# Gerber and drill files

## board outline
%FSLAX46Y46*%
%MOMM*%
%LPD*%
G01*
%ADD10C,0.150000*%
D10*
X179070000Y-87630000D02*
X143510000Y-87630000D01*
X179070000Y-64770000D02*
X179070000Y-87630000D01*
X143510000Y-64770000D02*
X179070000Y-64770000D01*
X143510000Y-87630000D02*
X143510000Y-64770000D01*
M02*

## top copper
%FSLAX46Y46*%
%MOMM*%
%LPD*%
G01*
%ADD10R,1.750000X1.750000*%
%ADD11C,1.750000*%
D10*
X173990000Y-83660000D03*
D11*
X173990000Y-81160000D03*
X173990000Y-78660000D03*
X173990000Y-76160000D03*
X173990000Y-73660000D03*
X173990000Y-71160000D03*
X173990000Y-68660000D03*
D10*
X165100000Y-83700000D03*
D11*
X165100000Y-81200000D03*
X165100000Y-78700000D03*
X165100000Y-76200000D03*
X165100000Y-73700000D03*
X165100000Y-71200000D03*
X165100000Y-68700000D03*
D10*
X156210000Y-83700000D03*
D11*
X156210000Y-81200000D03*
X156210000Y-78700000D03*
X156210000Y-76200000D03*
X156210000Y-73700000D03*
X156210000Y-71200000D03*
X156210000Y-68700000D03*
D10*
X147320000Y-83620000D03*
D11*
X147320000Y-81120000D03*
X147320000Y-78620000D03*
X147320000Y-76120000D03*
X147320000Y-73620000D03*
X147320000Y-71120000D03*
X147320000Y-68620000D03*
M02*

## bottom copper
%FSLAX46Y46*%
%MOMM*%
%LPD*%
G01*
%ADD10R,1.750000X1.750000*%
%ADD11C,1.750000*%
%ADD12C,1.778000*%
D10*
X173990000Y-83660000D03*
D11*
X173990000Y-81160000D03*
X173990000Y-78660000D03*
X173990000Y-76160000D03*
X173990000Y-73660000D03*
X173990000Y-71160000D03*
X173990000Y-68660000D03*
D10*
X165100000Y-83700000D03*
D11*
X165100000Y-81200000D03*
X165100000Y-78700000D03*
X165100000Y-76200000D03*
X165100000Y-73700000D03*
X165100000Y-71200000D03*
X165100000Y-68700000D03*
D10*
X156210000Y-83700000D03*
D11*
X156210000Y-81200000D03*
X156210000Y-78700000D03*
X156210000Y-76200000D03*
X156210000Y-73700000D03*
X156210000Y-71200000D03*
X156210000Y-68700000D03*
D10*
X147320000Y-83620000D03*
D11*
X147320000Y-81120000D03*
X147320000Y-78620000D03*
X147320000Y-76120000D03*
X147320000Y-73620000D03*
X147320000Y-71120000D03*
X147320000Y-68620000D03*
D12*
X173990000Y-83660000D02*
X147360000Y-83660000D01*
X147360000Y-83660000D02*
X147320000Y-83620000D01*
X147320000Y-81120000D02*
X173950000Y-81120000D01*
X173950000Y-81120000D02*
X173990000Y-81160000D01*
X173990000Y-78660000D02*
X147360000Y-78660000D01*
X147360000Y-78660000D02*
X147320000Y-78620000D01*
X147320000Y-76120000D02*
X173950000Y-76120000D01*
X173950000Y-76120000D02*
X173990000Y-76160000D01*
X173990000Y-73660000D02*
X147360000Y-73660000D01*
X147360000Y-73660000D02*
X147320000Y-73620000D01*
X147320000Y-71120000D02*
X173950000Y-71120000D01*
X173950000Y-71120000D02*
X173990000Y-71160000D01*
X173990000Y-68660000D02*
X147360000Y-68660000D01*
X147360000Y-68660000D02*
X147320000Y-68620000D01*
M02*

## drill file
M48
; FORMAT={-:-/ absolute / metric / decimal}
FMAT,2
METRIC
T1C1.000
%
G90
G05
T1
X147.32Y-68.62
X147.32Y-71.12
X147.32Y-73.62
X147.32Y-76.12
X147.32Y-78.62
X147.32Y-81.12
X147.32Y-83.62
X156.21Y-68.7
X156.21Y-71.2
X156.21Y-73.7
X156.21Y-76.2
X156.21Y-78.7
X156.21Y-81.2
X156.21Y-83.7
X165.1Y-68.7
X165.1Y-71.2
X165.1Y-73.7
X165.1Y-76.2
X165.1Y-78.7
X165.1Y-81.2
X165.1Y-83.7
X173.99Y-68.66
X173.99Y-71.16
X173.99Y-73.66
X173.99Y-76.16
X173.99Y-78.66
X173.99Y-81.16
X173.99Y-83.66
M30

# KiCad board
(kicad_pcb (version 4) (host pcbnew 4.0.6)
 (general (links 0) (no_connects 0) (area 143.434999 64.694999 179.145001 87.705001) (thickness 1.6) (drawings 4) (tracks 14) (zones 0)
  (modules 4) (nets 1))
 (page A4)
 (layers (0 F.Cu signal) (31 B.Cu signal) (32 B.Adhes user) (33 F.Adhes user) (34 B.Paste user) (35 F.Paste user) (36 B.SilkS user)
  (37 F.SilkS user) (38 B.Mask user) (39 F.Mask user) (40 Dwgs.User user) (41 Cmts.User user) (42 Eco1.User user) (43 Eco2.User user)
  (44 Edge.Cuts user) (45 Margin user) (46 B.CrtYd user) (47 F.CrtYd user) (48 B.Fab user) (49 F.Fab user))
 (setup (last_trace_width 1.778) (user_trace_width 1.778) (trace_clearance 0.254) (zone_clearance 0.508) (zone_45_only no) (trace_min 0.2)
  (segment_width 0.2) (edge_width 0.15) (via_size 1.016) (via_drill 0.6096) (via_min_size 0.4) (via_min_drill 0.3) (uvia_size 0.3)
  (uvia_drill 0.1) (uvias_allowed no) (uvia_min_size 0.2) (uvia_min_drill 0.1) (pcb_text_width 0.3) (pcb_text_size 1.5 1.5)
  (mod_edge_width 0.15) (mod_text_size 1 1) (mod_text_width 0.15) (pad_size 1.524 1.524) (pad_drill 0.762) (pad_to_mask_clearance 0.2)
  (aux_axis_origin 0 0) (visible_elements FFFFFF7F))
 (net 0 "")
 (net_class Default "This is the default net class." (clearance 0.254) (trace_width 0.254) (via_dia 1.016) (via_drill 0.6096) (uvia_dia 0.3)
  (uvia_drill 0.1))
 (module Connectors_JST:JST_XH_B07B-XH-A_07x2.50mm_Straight (layer F.Cu) (at 173.99 83.66 90)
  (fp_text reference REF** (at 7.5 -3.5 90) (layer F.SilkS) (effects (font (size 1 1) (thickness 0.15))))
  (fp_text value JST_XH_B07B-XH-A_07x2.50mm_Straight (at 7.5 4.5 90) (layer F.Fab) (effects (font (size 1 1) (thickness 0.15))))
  (pad 1 thru_hole rect (at 0 0 90) (size 1.75 1.75) (drill 1) (layers *.Cu *.Mask))
  (pad 2 thru_hole circle (at 2.5 0 90) (size 1.75 1.75) (drill 1) (layers *.Cu *.Mask))
  (pad 3 thru_hole circle (at 5 0 90) (size 1.75 1.75) (drill 1) (layers *.Cu *.Mask))
  (pad 4 thru_hole circle (at 7.5 0 90) (size 1.75 1.75) (drill 1) (layers *.Cu *.Mask))
  (pad 5 thru_hole circle (at 10 0 90) (size 1.75 1.75) (drill 1) (layers *.Cu *.Mask))
  (pad 6 thru_hole circle (at 12.5 0 90) (size 1.75 1.75) (drill 1) (layers *.Cu *.Mask))
  (pad 7 thru_hole circle (at 15 0 90) (size 1.75 1.75) (drill 1) (layers *.Cu *.Mask)))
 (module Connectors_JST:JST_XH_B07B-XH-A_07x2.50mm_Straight (layer F.Cu) (at 165.1 83.7 90)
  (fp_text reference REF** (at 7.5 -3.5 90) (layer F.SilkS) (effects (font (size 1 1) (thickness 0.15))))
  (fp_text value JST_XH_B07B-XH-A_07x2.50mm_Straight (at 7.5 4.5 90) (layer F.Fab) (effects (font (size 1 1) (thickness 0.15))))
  (pad 1 thru_hole rect (at 0 0 90) (size 1.75 1.75) (drill 1) (layers *.Cu *.Mask))
  (pad 2 thru_hole circle (at 2.5 0 90) (size 1.75 1.75) (drill 1) (layers *.Cu *.Mask))
  (pad 3 thru_hole circle (at 5 0 90) (size 1.75 1.75) (drill 1) (layers *.Cu *.Mask))
  (pad 4 thru_hole circle (at 7.5 0 90) (size 1.75 1.75) (drill 1) (layers *.Cu *.Mask))
  (pad 5 thru_hole circle (at 10 0 90) (size 1.75 1.75) (drill 1) (layers *.Cu *.Mask))
  (pad 6 thru_hole circle (at 12.5 0 90) (size 1.75 1.75) (drill 1) (layers *.Cu *.Mask))
  (pad 7 thru_hole circle (at 15 0 90) (size 1.75 1.75) (drill 1) (layers *.Cu *.Mask)))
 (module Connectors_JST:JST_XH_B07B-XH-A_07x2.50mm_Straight (layer F.Cu) (at 156.21 83.7 90)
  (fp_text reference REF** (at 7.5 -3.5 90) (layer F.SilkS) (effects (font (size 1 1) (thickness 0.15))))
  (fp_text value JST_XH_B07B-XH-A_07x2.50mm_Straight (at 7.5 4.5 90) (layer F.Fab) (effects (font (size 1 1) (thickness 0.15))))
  (pad 1 thru_hole rect (at 0 0 90) (size 1.75 1.75) (drill 1) (layers *.Cu *.Mask))
  (pad 2 thru_hole circle (at 2.5 0 90) (size 1.75 1.75) (drill 1) (layers *.Cu *.Mask))
  (pad 3 thru_hole circle (at 5 0 90) (size 1.75 1.75) (drill 1) (layers *.Cu *.Mask))
  (pad 4 thru_hole circle (at 7.5 0 90) (size 1.75 1.75) (drill 1) (layers *.Cu *.Mask))
  (pad 5 thru_hole circle (at 10 0 90) (size 1.75 1.75) (drill 1) (layers *.Cu *.Mask))
  (pad 6 thru_hole circle (at 12.5 0 90) (size 1.75 1.75) (drill 1) (layers *.Cu *.Mask))
  (pad 7 thru_hole circle (at 15 0 90) (size 1.75 1.75) (drill 1) (layers *.Cu *.Mask)))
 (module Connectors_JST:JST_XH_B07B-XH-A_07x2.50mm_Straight (layer F.Cu) (at 147.32 83.62 90)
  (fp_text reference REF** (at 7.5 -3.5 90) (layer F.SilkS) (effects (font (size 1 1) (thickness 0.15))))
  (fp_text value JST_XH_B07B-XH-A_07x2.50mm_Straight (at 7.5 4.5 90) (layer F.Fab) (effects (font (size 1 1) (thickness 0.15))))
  (pad 1 thru_hole rect (at 0 0 90) (size 1.75 1.75) (drill 1) (layers *.Cu *.Mask))
  (pad 2 thru_hole circle (at 2.5 0 90) (size 1.75 1.75) (drill 1) (layers *.Cu *.Mask))
  (pad 3 thru_hole circle (at 5 0 90) (size 1.75 1.75) (drill 1) (layers *.Cu *.Mask))
  (pad 4 thru_hole circle (at 7.5 0 90) (size 1.75 1.75) (drill 1) (layers *.Cu *.Mask))
  (pad 5 thru_hole circle (at 10 0 90) (size 1.75 1.75) (drill 1) (layers *.Cu *.Mask))
  (pad 6 thru_hole circle (at 12.5 0 90) (size 1.75 1.75) (drill 1) (layers *.Cu *.Mask))
  (pad 7 thru_hole circle (at 15 0 90) (size 1.75 1.75) (drill 1) (layers *.Cu *.Mask)))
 (gr_line (start 179.07 87.63) (end 143.51 87.63) (layer Edge.Cuts) (width 0.15))
 (gr_line (start 179.07 64.77) (end 179.07 87.63) (layer Edge.Cuts) (width 0.15))
 (gr_line (start 143.51 64.77) (end 179.07 64.77) (layer Edge.Cuts) (width 0.15))
 (gr_line (start 143.51 87.63) (end 143.51 64.77) (layer Edge.Cuts) (width 0.15))
 (segment (start 173.99 83.66) (end 147.36 83.66) (width 1.778) (layer B.Cu) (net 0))
 (segment (start 147.36 83.66) (end 147.32 83.62) (width 1.778) (layer B.Cu) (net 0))
 (segment (start 147.32 81.12) (end 173.95 81.12) (width 1.778) (layer B.Cu) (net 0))
 (segment (start 173.95 81.12) (end 173.99 81.16) (width 1.778) (layer B.Cu) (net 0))
 (segment (start 173.99 78.66) (end 147.36 78.66) (width 1.778) (layer B.Cu) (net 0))
 (segment (start 147.36 78.66) (end 147.32 78.62) (width 1.778) (layer B.Cu) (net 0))
 (segment (start 147.32 76.12) (end 173.95 76.12) (width 1.778) (layer B.Cu) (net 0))
 (segment (start 173.95 76.12) (end 173.99 76.16) (width 1.778) (layer B.Cu) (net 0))
 (segment (start 173.99 73.66) (end 147.36 73.66) (width 1.778) (layer B.Cu) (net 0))
 (segment (start 147.36 73.66) (end 147.32 73.62) (width 1.778) (layer B.Cu) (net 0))
 (segment (start 147.32 71.12) (end 173.95 71.12) (width 1.778) (layer B.Cu) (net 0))
 (segment (start 173.95 71.12) (end 173.99 71.16) (width 1.778) (layer B.Cu) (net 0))
 (segment (start 173.99 68.66) (end 147.36 68.66) (width 1.778) (layer B.Cu) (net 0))
 (segment (start 147.36 68.66) (end 147.32 68.62) (width 1.778) (layer B.Cu) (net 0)))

